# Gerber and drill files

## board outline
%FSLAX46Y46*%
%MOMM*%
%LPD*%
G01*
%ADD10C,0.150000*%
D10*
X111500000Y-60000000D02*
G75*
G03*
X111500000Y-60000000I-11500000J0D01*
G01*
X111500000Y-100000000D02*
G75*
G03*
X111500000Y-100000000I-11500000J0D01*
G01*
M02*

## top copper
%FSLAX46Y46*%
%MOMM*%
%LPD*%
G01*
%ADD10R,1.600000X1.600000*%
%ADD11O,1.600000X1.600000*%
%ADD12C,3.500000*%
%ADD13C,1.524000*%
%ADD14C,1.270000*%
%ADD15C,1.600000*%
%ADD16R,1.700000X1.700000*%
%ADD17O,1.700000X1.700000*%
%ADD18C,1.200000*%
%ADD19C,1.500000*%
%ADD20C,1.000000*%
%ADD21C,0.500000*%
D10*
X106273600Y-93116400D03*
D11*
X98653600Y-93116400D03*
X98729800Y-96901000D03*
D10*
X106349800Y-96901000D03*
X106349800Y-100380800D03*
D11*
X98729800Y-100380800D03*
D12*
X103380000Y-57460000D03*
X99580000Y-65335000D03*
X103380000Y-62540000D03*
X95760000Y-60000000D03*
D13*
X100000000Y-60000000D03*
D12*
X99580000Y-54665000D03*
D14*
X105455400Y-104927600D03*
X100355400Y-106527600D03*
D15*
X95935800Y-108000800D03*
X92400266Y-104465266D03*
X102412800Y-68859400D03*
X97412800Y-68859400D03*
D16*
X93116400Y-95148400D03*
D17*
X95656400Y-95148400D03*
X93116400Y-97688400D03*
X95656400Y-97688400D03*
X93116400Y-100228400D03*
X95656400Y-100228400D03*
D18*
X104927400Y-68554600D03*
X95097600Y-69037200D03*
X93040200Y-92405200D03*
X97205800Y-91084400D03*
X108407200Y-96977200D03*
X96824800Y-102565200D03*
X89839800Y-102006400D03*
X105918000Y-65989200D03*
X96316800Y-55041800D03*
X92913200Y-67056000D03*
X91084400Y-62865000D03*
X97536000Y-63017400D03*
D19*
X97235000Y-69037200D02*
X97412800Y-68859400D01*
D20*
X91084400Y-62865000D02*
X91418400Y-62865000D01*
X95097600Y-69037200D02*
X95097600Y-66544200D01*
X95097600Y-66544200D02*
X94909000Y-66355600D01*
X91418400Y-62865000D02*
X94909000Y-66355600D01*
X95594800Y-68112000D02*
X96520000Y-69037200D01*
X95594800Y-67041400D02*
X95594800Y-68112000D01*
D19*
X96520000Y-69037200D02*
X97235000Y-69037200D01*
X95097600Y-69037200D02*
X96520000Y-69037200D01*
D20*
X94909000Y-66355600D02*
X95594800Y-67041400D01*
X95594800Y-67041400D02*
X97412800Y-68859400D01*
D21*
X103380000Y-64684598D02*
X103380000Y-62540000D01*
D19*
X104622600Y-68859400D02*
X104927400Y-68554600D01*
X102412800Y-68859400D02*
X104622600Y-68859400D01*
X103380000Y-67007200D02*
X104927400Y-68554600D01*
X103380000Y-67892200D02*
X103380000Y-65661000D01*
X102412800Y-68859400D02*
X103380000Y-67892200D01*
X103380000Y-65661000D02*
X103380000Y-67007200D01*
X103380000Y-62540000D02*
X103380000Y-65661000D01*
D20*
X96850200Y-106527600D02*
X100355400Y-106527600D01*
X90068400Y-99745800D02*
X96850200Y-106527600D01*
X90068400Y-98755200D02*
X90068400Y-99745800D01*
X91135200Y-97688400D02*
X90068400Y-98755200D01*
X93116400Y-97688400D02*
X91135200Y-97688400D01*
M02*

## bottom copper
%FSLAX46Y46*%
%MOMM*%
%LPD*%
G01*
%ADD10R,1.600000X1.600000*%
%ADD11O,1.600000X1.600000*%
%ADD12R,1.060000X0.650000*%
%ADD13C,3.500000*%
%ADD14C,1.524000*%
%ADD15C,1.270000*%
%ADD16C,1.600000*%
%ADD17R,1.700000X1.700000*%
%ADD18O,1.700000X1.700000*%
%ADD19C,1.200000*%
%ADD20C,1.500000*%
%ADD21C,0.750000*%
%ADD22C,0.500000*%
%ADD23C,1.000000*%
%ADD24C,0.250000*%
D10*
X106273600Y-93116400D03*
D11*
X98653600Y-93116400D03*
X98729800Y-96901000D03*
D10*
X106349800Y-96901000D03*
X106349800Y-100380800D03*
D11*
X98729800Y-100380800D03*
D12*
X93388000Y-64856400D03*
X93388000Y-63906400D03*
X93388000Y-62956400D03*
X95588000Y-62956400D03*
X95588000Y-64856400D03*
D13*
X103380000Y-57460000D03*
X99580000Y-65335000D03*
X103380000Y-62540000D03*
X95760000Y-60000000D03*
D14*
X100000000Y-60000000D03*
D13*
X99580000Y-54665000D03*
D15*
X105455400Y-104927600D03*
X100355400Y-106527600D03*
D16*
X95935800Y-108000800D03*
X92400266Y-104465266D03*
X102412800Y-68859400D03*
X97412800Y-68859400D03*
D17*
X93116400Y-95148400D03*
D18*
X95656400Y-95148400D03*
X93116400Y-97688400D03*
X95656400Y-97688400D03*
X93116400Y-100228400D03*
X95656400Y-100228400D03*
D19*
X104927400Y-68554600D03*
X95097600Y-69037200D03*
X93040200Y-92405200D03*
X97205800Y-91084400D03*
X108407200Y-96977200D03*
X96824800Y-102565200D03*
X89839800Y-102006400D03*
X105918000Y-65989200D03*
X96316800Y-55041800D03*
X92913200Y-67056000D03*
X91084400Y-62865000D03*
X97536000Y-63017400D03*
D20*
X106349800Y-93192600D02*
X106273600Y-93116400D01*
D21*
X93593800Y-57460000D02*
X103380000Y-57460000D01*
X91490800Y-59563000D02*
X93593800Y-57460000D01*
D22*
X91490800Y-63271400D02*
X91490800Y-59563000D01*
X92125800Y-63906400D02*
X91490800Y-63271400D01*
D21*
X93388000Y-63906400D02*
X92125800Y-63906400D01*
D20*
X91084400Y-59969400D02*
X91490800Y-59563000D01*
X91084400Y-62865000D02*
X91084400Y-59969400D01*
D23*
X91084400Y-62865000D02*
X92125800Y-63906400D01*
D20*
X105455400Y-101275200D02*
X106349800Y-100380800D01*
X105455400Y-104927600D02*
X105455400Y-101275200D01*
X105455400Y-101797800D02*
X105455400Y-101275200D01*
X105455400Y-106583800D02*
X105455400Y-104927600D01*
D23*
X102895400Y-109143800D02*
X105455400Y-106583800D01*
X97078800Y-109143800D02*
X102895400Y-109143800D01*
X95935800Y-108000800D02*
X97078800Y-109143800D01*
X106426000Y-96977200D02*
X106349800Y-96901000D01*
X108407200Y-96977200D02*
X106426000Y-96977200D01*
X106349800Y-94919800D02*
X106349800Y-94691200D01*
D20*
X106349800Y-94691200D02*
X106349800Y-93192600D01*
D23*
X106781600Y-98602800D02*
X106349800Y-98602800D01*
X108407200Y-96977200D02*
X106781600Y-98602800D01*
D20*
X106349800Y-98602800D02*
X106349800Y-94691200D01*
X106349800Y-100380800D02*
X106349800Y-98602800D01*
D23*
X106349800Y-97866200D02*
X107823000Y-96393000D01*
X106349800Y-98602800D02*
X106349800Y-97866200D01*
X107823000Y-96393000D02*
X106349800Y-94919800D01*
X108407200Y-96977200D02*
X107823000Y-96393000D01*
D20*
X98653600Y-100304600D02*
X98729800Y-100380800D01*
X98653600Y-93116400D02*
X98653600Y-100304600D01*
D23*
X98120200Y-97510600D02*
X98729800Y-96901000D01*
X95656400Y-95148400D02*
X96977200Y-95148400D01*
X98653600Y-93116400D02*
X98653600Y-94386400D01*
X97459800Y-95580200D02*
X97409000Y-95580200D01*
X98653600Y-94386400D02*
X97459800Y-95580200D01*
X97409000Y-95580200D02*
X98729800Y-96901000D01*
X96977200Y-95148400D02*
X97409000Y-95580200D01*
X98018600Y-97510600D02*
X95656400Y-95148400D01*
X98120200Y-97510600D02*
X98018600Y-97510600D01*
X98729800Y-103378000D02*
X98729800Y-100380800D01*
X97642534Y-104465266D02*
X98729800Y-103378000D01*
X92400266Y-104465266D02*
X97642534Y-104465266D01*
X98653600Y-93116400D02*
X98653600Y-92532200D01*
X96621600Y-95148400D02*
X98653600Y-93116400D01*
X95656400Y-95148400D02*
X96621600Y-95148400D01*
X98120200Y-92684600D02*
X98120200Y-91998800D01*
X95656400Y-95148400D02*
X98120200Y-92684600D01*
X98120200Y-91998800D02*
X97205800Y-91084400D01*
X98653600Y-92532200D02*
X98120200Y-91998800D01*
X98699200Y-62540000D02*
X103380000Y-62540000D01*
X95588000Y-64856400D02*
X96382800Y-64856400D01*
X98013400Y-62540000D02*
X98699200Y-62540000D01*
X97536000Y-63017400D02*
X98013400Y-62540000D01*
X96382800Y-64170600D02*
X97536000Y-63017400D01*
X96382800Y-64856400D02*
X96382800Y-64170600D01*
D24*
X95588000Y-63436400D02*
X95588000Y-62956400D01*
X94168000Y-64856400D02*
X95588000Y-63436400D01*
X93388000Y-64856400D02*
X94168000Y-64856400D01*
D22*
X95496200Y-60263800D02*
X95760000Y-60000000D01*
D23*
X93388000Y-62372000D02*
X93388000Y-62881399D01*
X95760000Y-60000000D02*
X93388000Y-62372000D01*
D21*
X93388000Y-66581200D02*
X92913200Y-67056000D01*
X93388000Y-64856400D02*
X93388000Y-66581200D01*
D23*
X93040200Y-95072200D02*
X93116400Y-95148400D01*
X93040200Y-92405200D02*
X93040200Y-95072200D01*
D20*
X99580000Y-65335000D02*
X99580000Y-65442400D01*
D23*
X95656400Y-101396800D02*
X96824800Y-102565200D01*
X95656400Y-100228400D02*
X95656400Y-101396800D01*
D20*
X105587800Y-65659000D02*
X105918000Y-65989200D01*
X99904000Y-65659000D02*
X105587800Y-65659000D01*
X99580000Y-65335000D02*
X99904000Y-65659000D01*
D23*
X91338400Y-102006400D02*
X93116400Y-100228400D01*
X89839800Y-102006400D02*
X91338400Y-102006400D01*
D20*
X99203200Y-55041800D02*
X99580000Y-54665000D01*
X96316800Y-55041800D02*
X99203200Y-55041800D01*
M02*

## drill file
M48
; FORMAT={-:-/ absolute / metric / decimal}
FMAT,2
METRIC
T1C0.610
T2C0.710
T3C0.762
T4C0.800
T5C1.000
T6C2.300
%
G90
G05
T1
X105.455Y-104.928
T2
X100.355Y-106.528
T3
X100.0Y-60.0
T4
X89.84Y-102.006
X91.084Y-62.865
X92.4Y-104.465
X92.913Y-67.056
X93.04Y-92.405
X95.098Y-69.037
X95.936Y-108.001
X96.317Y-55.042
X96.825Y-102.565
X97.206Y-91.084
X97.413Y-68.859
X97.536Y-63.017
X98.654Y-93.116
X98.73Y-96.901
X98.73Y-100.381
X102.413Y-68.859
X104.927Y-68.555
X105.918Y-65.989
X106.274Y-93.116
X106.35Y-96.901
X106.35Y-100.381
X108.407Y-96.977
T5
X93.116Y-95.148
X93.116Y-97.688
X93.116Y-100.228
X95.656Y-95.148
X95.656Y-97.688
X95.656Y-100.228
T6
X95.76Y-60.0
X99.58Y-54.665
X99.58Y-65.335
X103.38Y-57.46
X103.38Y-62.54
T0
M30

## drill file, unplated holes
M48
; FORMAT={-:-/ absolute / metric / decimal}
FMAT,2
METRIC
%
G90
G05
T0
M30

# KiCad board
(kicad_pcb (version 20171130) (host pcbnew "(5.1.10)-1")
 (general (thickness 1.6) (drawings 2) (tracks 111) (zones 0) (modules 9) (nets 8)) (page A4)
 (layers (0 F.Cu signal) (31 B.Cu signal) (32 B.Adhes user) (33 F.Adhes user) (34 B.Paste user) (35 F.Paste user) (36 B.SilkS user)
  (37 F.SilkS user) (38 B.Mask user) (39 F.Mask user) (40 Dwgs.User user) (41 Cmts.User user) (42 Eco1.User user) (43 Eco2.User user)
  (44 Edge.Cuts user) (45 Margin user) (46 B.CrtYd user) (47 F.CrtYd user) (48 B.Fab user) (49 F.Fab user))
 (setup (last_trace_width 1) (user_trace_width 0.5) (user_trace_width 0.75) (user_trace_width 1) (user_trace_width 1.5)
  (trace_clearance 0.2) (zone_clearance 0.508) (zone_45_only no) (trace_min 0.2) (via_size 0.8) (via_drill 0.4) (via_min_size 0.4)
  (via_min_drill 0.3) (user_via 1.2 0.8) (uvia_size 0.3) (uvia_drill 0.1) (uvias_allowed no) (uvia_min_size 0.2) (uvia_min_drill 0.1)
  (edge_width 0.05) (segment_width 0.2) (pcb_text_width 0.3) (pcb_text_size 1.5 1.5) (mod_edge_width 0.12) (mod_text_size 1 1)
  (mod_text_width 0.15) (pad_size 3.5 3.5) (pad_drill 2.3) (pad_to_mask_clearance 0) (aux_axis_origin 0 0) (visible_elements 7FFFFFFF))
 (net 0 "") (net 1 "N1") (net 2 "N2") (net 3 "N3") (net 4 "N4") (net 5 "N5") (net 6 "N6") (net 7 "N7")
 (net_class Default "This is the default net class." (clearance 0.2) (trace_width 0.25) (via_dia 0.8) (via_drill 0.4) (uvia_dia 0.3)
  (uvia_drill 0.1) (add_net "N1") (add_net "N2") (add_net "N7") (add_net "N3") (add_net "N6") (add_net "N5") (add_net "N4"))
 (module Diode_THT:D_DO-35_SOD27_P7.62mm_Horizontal (layer B.Cu) (at 106.2736 93.1164 180)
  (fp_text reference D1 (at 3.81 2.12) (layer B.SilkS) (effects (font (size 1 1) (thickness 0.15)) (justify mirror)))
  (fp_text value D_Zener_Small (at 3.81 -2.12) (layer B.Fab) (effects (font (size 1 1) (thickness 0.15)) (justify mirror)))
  (pad 1 thru_hole rect (at 0 0 180) (size 1.6 1.6) (drill 0.8) (layers *.Cu *.Mask) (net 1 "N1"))
  (pad 2 thru_hole oval (at 7.62 0 180) (size 1.6 1.6) (drill 0.8) (layers *.Cu *.Mask) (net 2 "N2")))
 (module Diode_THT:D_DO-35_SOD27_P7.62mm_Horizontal (layer B.Cu) (at 106.3498 96.901 180)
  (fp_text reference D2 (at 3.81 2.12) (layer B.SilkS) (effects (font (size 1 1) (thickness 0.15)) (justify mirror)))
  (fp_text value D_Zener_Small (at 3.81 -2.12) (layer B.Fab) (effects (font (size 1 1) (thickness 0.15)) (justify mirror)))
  (pad 2 thru_hole oval (at 7.62 0 180) (size 1.6 1.6) (drill 0.8) (layers *.Cu *.Mask) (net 2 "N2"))
  (pad 1 thru_hole rect (at 0 0 180) (size 1.6 1.6) (drill 0.8) (layers *.Cu *.Mask) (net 1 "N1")))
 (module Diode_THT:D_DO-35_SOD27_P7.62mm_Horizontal (layer B.Cu) (at 106.3498 100.3808 180)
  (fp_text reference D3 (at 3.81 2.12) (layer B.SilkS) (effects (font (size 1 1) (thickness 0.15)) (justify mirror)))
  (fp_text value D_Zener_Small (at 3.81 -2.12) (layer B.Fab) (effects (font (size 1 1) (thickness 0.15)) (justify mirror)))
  (pad 1 thru_hole rect (at 0 0 180) (size 1.6 1.6) (drill 0.8) (layers *.Cu *.Mask) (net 1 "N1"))
  (pad 2 thru_hole oval (at 7.62 0 180) (size 1.6 1.6) (drill 0.8) (layers *.Cu *.Mask) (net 2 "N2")))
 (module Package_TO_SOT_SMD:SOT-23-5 (layer B.Cu) (at 94.488 63.9064)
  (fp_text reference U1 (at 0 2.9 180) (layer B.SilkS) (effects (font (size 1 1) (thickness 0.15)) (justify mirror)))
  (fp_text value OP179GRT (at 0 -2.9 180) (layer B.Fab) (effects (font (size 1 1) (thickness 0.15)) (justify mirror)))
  (pad 1 smd rect (at -1.1 0.95) (size 1.06 0.65) (layers B.Cu B.Paste B.Mask) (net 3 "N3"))
  (pad 2 smd rect (at -1.1 0) (size 1.06 0.65) (layers B.Cu B.Paste B.Mask) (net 1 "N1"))
  (pad 3 smd rect (at -1.1 -0.95) (size 1.06 0.65) (layers B.Cu B.Paste B.Mask) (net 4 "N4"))
  (pad 4 smd rect (at 1.1 -0.95) (size 1.06 0.65) (layers B.Cu B.Paste B.Mask) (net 3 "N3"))
  (pad 5 smd rect (at 1.1 0.95) (size 1.06 0.65) (layers B.Cu B.Paste B.Mask) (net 2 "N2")))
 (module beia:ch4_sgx (layer F.Cu) (at 100 60)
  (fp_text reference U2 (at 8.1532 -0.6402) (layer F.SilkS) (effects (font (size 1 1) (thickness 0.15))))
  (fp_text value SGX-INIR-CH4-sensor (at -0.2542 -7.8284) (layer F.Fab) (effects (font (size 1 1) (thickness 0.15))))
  (pad 2 thru_hole circle (at 3.38 -2.54) (size 3.5 3.5) (drill 2.3) (layers *.Cu *.Mask) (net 1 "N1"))
  (pad 4 thru_hole circle (at -0.42 5.335) (size 3.5 3.5) (drill 2.3) (layers *.Cu *.Mask) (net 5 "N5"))
  (pad 3 thru_hole circle (at 3.38 2.54) (size 3.5 3.5) (drill 2.3) (layers *.Cu *.Mask) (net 2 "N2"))
  (pad 5 thru_hole circle (at -4.24 0) (size 3.5 3.5) (drill 2.3) (layers *.Cu *.Mask) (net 4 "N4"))
  (pad P1 thru_hole circle (at 0 0) (size 1.524 1.524) (drill 0.762) (layers *.Cu *.Mask))
  (pad 1 thru_hole circle (at -0.42 -5.335) (size 3.5 3.5) (drill 2.3) (layers *.Cu *.Mask) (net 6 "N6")))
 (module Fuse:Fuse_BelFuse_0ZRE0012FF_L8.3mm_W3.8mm (layer B.Cu) (at 100.3554 106.5276)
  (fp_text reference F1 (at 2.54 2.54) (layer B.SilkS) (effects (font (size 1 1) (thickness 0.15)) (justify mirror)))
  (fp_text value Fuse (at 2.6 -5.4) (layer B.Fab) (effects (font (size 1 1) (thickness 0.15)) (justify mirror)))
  (pad 2 thru_hole circle (at 5.1 -1.6) (size 1.27 1.27) (drill 0.61) (layers *.Cu *.Mask) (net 1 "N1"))
  (pad 1 thru_hole circle (at 0 0) (size 1.27 1.27) (drill 0.71) (layers *.Cu *.Mask) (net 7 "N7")))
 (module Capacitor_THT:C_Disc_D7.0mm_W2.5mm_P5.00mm (layer F.Cu) (at 95.9358 108.0008 135)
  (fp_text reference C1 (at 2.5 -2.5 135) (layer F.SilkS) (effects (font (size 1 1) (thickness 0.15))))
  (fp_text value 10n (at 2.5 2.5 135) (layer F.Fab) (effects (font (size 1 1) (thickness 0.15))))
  (pad 1 thru_hole circle (at 0 0 135) (size 1.6 1.6) (drill 0.8) (layers *.Cu *.Mask) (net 1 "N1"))
  (pad 2 thru_hole circle (at 5 0 135) (size 1.6 1.6) (drill 0.8) (layers *.Cu *.Mask) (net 2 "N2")))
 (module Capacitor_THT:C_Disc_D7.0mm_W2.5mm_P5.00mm (layer F.Cu) (at 102.4128 68.8594 180)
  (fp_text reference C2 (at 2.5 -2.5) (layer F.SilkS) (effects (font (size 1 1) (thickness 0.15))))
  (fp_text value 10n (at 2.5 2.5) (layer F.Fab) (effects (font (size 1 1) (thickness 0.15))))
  (pad 1 thru_hole circle (at 0 0 180) (size 1.6 1.6) (drill 0.8) (layers *.Cu *.Mask) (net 2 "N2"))
  (pad 2 thru_hole circle (at 5 0 180) (size 1.6 1.6) (drill 0.8) (layers *.Cu *.Mask) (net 1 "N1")))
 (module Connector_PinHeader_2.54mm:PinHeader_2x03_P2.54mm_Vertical (layer F.Cu) (at 93.1164 95.1484)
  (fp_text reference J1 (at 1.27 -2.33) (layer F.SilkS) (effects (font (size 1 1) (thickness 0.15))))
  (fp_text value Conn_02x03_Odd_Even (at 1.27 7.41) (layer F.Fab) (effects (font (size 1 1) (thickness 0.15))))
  (pad 1 thru_hole rect (at 0 0) (size 1.7 1.7) (drill 1) (layers *.Cu *.Mask) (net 3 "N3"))
  (pad 2 thru_hole oval (at 2.54 0) (size 1.7 1.7) (drill 1) (layers *.Cu *.Mask) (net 2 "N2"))
  (pad 3 thru_hole oval (at 0 2.54) (size 1.7 1.7) (drill 1) (layers *.Cu *.Mask) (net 7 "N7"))
  (pad 4 thru_hole oval (at 2.54 2.54) (size 1.7 1.7) (drill 1) (layers *.Cu *.Mask) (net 3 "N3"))
  (pad 5 thru_hole oval (at 0 5.08) (size 1.7 1.7) (drill 1) (layers *.Cu *.Mask) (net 6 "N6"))
  (pad 6 thru_hole oval (at 2.54 5.08) (size 1.7 1.7) (drill 1) (layers *.Cu *.Mask) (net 5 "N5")))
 (gr_circle (center 100 60) (end 111.5 60) (layer Edge.Cuts) (width 0.15))
 (gr_circle (center 100 100) (end 111.5 100) (layer Edge.Cuts) (width 0.15))
 (via (at 104.9274 68.5546) (size 1.2) (drill 0.8) (layers F.Cu B.Cu) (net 2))
 (via (at 95.0976 69.0372) (size 1.2) (drill 0.8) (layers F.Cu B.Cu) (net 1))
 (via (at 93.0402 92.4052) (size 1.2) (drill 0.8) (layers F.Cu B.Cu) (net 3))
 (via (at 97.2058 91.0844) (size 1.2) (drill 0.8) (layers F.Cu B.Cu) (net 2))
 (via (at 108.4072 96.9772) (size 1.2) (drill 0.8) (layers F.Cu B.Cu) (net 1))
 (via (at 96.8248 102.5652) (size 1.2) (drill 0.8) (layers F.Cu B.Cu) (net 5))
 (via (at 89.8398 102.0064) (size 1.2) (drill 0.8) (layers F.Cu B.Cu) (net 6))
 (via (at 105.918 65.9892) (size 1.2) (drill 0.8) (layers F.Cu B.Cu) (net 5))
 (via (at 96.3168 55.0418) (size 1.2) (drill 0.8) (layers F.Cu B.Cu) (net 6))
 (via (at 92.9132 67.056) (size 1.2) (drill 0.8) (layers F.Cu B.Cu) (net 3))
 (via (at 91.0844 62.865) (size 1.2) (drill 0.8) (layers F.Cu B.Cu) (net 1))
 (segment (start 106.3498 93.1926) (end 106.2736 93.1164) (width 1.5) (layer B.Cu) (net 1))
 (segment (start 93.5938 57.46) (end 103.38 57.46) (width 0.75) (layer B.Cu) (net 1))
 (segment (start 91.4908 59.563) (end 93.5938 57.46) (width 0.75) (layer B.Cu) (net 1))
 (segment (start 91.4908 63.2714) (end 91.4908 59.563) (width 0.5) (layer B.Cu) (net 1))
 (segment (start 92.1258 63.9064) (end 91.4908 63.2714) (width 0.5) (layer B.Cu) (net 1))
 (segment (start 93.388 63.9064) (end 92.1258 63.9064) (width 0.75) (layer B.Cu) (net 1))
 (segment (start 91.0844 59.9694) (end 91.4908 59.563) (width 1.5) (layer B.Cu) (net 1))
 (segment (start 91.0844 62.865) (end 91.0844 59.9694) (width 1.5) (layer B.Cu) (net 1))
 (segment (start 91.0844 62.865) (end 92.1258 63.9064) (width 1) (layer B.Cu) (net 1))
 (segment (start 105.4554 101.2752) (end 106.3498 100.3808) (width 1.5) (layer B.Cu) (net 1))
 (segment (start 105.4554 104.9276) (end 105.4554 101.2752) (width 1.5) (layer B.Cu) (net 1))
 (segment (start 105.4554 101.7978) (end 105.4554 101.2752) (width 1.5) (layer B.Cu) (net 1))
 (segment (start 105.4554 106.5838) (end 105.4554 104.9276) (width 1.5) (layer B.Cu) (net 1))
 (segment (start 102.8954 109.1438) (end 105.4554 106.5838) (width 1) (layer B.Cu) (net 1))
 (segment (start 97.0788 109.1438) (end 102.8954 109.1438) (width 1) (layer B.Cu) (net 1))
 (segment (start 95.9358 108.0008) (end 97.0788 109.1438) (width 1) (layer B.Cu) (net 1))
 (segment (start 106.426 96.9772) (end 106.3498 96.901) (width 1) (layer B.Cu) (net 1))
 (segment (start 108.4072 96.9772) (end 106.426 96.9772) (width 1) (layer B.Cu) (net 1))
 (segment (start 106.3498 94.9198) (end 106.3498 94.6912) (width 1) (layer B.Cu) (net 1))
 (segment (start 106.3498 94.6912) (end 106.3498 93.1926) (width 1.5) (layer B.Cu) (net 1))
 (segment (start 106.7816 98.6028) (end 106.3498 98.6028) (width 1) (layer B.Cu) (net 1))
 (segment (start 108.4072 96.9772) (end 106.7816 98.6028) (width 1) (layer B.Cu) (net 1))
 (segment (start 106.3498 98.6028) (end 106.3498 94.6912) (width 1.5) (layer B.Cu) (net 1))
 (segment (start 106.3498 100.3808) (end 106.3498 98.6028) (width 1.5) (layer B.Cu) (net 1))
 (segment (start 106.3498 97.8662) (end 107.823 96.393) (width 1) (layer B.Cu) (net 1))
 (segment (start 106.3498 98.6028) (end 106.3498 97.8662) (width 1) (layer B.Cu) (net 1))
 (segment (start 107.823 96.393) (end 106.3498 94.9198) (width 1) (layer B.Cu) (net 1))
 (segment (start 108.4072 96.9772) (end 107.823 96.393) (width 1) (layer B.Cu) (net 1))
 (segment (start 97.235 69.0372) (end 97.4128 68.8594) (width 1.5) (layer F.Cu) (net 1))
 (segment (start 91.0844 62.865) (end 91.4184 62.865) (width 1) (layer F.Cu) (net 1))
 (segment (start 95.0976 69.0372) (end 95.0976 66.5442) (width 1) (layer F.Cu) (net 1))
 (segment (start 95.0976 66.5442) (end 94.909 66.3556) (width 1) (layer F.Cu) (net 1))
 (segment (start 91.4184 62.865) (end 94.909 66.3556) (width 1) (layer F.Cu) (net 1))
 (segment (start 95.5948 68.112) (end 96.52 69.0372) (width 1) (layer F.Cu) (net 1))
 (segment (start 95.5948 67.0414) (end 95.5948 68.112) (width 1) (layer F.Cu) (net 1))
 (segment (start 96.52 69.0372) (end 97.235 69.0372) (width 1.5) (layer F.Cu) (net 1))
 (segment (start 95.0976 69.0372) (end 96.52 69.0372) (width 1.5) (layer F.Cu) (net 1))
 (segment (start 94.909 66.3556) (end 95.5948 67.0414) (width 1) (layer F.Cu) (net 1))
 (segment (start 95.5948 67.0414) (end 97.4128 68.8594) (width 1) (layer F.Cu) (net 1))
 (via (at 97.536 63.0174) (size 1.2) (drill 0.8) (layers F.Cu B.Cu) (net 2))
 (segment (start 98.6536 100.3046) (end 98.7298 100.3808) (width 1.5) (layer B.Cu) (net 2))
 (segment (start 98.6536 93.1164) (end 98.6536 100.3046) (width 1.5) (layer B.Cu) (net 2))
 (segment (start 103.38 64.684598) (end 103.38 62.54) (width 0.5) (layer F.Cu) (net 2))
 (segment (start 98.1202 97.5106) (end 98.7298 96.901) (width 1) (layer B.Cu) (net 2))
 (segment (start 95.6564 95.1484) (end 96.9772 95.1484) (width 1) (layer B.Cu) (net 2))
 (segment (start 98.6536 93.1164) (end 98.6536 94.3864) (width 1) (layer B.Cu) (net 2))
 (segment (start 97.4598 95.5802) (end 97.409 95.5802) (width 1) (layer B.Cu) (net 2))
 (segment (start 98.6536 94.3864) (end 97.4598 95.5802) (width 1) (layer B.Cu) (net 2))
 (segment (start 97.409 95.5802) (end 98.7298 96.901) (width 1) (layer B.Cu) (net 2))
 (segment (start 96.9772 95.1484) (end 97.409 95.5802) (width 1) (layer B.Cu) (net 2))
 (segment (start 98.0186 97.5106) (end 95.6564 95.1484) (width 1) (layer B.Cu) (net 2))
 (segment (start 98.1202 97.5106) (end 98.0186 97.5106) (width 1) (layer B.Cu) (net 2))
 (segment (start 98.7298 103.378) (end 98.7298 100.3808) (width 1) (layer B.Cu) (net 2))
 (segment (start 97.642534 104.465266) (end 98.7298 103.378) (width 1) (layer B.Cu) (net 2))
 (segment (start 92.400266 104.465266) (end 97.642534 104.465266) (width 1) (layer B.Cu) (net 2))
 (segment (start 98.6536 93.1164) (end 98.6536 92.5322) (width 1) (layer B.Cu) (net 2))
 (segment (start 96.6216 95.1484) (end 98.6536 93.1164) (width 1) (layer B.Cu) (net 2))
 (segment (start 95.6564 95.1484) (end 96.6216 95.1484) (width 1) (layer B.Cu) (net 2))
 (segment (start 98.1202 92.6846) (end 98.1202 91.9988) (width 1) (layer B.Cu) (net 2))
 (segment (start 95.6564 95.1484) (end 98.1202 92.6846) (width 1) (layer B.Cu) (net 2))
 (segment (start 98.1202 91.9988) (end 97.2058 91.0844) (width 1) (layer B.Cu) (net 2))
 (segment (start 98.6536 92.5322) (end 98.1202 91.9988) (width 1) (layer B.Cu) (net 2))
 (segment (start 104.6226 68.8594) (end 104.9274 68.5546) (width 1.5) (layer F.Cu) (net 2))
 (segment (start 102.4128 68.8594) (end 104.6226 68.8594) (width 1.5) (layer F.Cu) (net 2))
 (segment (start 103.38 67.0072) (end 104.9274 68.5546) (width 1.5) (layer F.Cu) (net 2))
 (segment (start 103.38 67.8922) (end 103.38 65.661) (width 1.5) (layer F.Cu) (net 2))
 (segment (start 102.4128 68.8594) (end 103.38 67.8922) (width 1.5) (layer F.Cu) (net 2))
 (segment (start 103.38 65.661) (end 103.38 67.0072) (width 1.5) (layer F.Cu) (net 2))
 (segment (start 103.38 62.54) (end 103.38 65.661) (width 1.5) (layer F.Cu) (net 2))
 (segment (start 98.6992 62.54) (end 103.38 62.54) (width 1) (layer B.Cu) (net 2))
 (segment (start 95.588 64.8564) (end 96.3828 64.8564) (width 1) (layer B.Cu) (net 2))
 (segment (start 98.0134 62.54) (end 98.6992 62.54) (width 1) (layer B.Cu) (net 2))
 (segment (start 97.536 63.0174) (end 98.0134 62.54) (width 1) (layer B.Cu) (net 2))
 (segment (start 96.3828 64.1706) (end 97.536 63.0174) (width 1) (layer B.Cu) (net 2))
 (segment (start 96.3828 64.8564) (end 96.3828 64.1706) (width 1) (layer B.Cu) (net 2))
 (segment (start 95.588 63.4364) (end 95.588 62.9564) (width 0.25) (layer B.Cu) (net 3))
 (segment (start 94.168 64.8564) (end 95.588 63.4364) (width 0.25) (layer B.Cu) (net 3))
 (segment (start 93.388 64.8564) (end 94.168 64.8564) (width 0.25) (layer B.Cu) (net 3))
 (segment (start 95.4962 60.2638) (end 95.76 60) (width 0.5) (layer B.Cu) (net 4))
 (segment (start 93.388 62.372) (end 93.388 62.881399) (width 1) (layer B.Cu) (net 4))
 (segment (start 95.76 60) (end 93.388 62.372) (width 1) (layer B.Cu) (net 4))
 (segment (start 96.8502 106.5276) (end 100.3554 106.5276) (width 1) (layer F.Cu) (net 7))
 (segment (start 90.0684 99.7458) (end 96.8502 106.5276) (width 1) (layer F.Cu) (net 7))
 (segment (start 90.0684 98.7552) (end 90.0684 99.7458) (width 1) (layer F.Cu) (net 7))
 (segment (start 91.1352 97.6884) (end 90.0684 98.7552) (width 1) (layer F.Cu) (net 7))
 (segment (start 93.1164 97.6884) (end 91.1352 97.6884) (width 1) (layer F.Cu) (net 7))
 (segment (start 93.388 66.5812) (end 92.9132 67.056) (width 0.75) (layer B.Cu) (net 3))
 (segment (start 93.388 64.8564) (end 93.388 66.5812) (width 0.75) (layer B.Cu) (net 3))
 (segment (start 93.0402 95.0722) (end 93.1164 95.1484) (width 1) (layer B.Cu) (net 3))
 (segment (start 93.0402 92.4052) (end 93.0402 95.0722) (width 1) (layer B.Cu) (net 3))
 (segment (start 99.58 65.335) (end 99.58 65.4424) (width 1.5) (layer B.Cu) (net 5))
 (segment (start 95.6564 101.3968) (end 96.8248 102.5652) (width 1) (layer B.Cu) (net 5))
 (segment (start 95.6564 100.2284) (end 95.6564 101.3968) (width 1) (layer B.Cu) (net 5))
 (segment (start 105.5878 65.659) (end 105.918 65.9892) (width 1.5) (layer B.Cu) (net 5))
 (segment (start 99.904 65.659) (end 105.5878 65.659) (width 1.5) (layer B.Cu) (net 5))
 (segment (start 99.58 65.335) (end 99.904 65.659) (width 1.5) (layer B.Cu) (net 5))
 (segment (start 91.3384 102.0064) (end 93.1164 100.2284) (width 1) (layer B.Cu) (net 6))
 (segment (start 89.8398 102.0064) (end 91.3384 102.0064) (width 1) (layer B.Cu) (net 6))
 (segment (start 99.2032 55.0418) (end 99.58 54.665) (width 1.5) (layer B.Cu) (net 6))
 (segment (start 96.3168 55.0418) (end 99.2032 55.0418) (width 1.5) (layer B.Cu) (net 6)))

